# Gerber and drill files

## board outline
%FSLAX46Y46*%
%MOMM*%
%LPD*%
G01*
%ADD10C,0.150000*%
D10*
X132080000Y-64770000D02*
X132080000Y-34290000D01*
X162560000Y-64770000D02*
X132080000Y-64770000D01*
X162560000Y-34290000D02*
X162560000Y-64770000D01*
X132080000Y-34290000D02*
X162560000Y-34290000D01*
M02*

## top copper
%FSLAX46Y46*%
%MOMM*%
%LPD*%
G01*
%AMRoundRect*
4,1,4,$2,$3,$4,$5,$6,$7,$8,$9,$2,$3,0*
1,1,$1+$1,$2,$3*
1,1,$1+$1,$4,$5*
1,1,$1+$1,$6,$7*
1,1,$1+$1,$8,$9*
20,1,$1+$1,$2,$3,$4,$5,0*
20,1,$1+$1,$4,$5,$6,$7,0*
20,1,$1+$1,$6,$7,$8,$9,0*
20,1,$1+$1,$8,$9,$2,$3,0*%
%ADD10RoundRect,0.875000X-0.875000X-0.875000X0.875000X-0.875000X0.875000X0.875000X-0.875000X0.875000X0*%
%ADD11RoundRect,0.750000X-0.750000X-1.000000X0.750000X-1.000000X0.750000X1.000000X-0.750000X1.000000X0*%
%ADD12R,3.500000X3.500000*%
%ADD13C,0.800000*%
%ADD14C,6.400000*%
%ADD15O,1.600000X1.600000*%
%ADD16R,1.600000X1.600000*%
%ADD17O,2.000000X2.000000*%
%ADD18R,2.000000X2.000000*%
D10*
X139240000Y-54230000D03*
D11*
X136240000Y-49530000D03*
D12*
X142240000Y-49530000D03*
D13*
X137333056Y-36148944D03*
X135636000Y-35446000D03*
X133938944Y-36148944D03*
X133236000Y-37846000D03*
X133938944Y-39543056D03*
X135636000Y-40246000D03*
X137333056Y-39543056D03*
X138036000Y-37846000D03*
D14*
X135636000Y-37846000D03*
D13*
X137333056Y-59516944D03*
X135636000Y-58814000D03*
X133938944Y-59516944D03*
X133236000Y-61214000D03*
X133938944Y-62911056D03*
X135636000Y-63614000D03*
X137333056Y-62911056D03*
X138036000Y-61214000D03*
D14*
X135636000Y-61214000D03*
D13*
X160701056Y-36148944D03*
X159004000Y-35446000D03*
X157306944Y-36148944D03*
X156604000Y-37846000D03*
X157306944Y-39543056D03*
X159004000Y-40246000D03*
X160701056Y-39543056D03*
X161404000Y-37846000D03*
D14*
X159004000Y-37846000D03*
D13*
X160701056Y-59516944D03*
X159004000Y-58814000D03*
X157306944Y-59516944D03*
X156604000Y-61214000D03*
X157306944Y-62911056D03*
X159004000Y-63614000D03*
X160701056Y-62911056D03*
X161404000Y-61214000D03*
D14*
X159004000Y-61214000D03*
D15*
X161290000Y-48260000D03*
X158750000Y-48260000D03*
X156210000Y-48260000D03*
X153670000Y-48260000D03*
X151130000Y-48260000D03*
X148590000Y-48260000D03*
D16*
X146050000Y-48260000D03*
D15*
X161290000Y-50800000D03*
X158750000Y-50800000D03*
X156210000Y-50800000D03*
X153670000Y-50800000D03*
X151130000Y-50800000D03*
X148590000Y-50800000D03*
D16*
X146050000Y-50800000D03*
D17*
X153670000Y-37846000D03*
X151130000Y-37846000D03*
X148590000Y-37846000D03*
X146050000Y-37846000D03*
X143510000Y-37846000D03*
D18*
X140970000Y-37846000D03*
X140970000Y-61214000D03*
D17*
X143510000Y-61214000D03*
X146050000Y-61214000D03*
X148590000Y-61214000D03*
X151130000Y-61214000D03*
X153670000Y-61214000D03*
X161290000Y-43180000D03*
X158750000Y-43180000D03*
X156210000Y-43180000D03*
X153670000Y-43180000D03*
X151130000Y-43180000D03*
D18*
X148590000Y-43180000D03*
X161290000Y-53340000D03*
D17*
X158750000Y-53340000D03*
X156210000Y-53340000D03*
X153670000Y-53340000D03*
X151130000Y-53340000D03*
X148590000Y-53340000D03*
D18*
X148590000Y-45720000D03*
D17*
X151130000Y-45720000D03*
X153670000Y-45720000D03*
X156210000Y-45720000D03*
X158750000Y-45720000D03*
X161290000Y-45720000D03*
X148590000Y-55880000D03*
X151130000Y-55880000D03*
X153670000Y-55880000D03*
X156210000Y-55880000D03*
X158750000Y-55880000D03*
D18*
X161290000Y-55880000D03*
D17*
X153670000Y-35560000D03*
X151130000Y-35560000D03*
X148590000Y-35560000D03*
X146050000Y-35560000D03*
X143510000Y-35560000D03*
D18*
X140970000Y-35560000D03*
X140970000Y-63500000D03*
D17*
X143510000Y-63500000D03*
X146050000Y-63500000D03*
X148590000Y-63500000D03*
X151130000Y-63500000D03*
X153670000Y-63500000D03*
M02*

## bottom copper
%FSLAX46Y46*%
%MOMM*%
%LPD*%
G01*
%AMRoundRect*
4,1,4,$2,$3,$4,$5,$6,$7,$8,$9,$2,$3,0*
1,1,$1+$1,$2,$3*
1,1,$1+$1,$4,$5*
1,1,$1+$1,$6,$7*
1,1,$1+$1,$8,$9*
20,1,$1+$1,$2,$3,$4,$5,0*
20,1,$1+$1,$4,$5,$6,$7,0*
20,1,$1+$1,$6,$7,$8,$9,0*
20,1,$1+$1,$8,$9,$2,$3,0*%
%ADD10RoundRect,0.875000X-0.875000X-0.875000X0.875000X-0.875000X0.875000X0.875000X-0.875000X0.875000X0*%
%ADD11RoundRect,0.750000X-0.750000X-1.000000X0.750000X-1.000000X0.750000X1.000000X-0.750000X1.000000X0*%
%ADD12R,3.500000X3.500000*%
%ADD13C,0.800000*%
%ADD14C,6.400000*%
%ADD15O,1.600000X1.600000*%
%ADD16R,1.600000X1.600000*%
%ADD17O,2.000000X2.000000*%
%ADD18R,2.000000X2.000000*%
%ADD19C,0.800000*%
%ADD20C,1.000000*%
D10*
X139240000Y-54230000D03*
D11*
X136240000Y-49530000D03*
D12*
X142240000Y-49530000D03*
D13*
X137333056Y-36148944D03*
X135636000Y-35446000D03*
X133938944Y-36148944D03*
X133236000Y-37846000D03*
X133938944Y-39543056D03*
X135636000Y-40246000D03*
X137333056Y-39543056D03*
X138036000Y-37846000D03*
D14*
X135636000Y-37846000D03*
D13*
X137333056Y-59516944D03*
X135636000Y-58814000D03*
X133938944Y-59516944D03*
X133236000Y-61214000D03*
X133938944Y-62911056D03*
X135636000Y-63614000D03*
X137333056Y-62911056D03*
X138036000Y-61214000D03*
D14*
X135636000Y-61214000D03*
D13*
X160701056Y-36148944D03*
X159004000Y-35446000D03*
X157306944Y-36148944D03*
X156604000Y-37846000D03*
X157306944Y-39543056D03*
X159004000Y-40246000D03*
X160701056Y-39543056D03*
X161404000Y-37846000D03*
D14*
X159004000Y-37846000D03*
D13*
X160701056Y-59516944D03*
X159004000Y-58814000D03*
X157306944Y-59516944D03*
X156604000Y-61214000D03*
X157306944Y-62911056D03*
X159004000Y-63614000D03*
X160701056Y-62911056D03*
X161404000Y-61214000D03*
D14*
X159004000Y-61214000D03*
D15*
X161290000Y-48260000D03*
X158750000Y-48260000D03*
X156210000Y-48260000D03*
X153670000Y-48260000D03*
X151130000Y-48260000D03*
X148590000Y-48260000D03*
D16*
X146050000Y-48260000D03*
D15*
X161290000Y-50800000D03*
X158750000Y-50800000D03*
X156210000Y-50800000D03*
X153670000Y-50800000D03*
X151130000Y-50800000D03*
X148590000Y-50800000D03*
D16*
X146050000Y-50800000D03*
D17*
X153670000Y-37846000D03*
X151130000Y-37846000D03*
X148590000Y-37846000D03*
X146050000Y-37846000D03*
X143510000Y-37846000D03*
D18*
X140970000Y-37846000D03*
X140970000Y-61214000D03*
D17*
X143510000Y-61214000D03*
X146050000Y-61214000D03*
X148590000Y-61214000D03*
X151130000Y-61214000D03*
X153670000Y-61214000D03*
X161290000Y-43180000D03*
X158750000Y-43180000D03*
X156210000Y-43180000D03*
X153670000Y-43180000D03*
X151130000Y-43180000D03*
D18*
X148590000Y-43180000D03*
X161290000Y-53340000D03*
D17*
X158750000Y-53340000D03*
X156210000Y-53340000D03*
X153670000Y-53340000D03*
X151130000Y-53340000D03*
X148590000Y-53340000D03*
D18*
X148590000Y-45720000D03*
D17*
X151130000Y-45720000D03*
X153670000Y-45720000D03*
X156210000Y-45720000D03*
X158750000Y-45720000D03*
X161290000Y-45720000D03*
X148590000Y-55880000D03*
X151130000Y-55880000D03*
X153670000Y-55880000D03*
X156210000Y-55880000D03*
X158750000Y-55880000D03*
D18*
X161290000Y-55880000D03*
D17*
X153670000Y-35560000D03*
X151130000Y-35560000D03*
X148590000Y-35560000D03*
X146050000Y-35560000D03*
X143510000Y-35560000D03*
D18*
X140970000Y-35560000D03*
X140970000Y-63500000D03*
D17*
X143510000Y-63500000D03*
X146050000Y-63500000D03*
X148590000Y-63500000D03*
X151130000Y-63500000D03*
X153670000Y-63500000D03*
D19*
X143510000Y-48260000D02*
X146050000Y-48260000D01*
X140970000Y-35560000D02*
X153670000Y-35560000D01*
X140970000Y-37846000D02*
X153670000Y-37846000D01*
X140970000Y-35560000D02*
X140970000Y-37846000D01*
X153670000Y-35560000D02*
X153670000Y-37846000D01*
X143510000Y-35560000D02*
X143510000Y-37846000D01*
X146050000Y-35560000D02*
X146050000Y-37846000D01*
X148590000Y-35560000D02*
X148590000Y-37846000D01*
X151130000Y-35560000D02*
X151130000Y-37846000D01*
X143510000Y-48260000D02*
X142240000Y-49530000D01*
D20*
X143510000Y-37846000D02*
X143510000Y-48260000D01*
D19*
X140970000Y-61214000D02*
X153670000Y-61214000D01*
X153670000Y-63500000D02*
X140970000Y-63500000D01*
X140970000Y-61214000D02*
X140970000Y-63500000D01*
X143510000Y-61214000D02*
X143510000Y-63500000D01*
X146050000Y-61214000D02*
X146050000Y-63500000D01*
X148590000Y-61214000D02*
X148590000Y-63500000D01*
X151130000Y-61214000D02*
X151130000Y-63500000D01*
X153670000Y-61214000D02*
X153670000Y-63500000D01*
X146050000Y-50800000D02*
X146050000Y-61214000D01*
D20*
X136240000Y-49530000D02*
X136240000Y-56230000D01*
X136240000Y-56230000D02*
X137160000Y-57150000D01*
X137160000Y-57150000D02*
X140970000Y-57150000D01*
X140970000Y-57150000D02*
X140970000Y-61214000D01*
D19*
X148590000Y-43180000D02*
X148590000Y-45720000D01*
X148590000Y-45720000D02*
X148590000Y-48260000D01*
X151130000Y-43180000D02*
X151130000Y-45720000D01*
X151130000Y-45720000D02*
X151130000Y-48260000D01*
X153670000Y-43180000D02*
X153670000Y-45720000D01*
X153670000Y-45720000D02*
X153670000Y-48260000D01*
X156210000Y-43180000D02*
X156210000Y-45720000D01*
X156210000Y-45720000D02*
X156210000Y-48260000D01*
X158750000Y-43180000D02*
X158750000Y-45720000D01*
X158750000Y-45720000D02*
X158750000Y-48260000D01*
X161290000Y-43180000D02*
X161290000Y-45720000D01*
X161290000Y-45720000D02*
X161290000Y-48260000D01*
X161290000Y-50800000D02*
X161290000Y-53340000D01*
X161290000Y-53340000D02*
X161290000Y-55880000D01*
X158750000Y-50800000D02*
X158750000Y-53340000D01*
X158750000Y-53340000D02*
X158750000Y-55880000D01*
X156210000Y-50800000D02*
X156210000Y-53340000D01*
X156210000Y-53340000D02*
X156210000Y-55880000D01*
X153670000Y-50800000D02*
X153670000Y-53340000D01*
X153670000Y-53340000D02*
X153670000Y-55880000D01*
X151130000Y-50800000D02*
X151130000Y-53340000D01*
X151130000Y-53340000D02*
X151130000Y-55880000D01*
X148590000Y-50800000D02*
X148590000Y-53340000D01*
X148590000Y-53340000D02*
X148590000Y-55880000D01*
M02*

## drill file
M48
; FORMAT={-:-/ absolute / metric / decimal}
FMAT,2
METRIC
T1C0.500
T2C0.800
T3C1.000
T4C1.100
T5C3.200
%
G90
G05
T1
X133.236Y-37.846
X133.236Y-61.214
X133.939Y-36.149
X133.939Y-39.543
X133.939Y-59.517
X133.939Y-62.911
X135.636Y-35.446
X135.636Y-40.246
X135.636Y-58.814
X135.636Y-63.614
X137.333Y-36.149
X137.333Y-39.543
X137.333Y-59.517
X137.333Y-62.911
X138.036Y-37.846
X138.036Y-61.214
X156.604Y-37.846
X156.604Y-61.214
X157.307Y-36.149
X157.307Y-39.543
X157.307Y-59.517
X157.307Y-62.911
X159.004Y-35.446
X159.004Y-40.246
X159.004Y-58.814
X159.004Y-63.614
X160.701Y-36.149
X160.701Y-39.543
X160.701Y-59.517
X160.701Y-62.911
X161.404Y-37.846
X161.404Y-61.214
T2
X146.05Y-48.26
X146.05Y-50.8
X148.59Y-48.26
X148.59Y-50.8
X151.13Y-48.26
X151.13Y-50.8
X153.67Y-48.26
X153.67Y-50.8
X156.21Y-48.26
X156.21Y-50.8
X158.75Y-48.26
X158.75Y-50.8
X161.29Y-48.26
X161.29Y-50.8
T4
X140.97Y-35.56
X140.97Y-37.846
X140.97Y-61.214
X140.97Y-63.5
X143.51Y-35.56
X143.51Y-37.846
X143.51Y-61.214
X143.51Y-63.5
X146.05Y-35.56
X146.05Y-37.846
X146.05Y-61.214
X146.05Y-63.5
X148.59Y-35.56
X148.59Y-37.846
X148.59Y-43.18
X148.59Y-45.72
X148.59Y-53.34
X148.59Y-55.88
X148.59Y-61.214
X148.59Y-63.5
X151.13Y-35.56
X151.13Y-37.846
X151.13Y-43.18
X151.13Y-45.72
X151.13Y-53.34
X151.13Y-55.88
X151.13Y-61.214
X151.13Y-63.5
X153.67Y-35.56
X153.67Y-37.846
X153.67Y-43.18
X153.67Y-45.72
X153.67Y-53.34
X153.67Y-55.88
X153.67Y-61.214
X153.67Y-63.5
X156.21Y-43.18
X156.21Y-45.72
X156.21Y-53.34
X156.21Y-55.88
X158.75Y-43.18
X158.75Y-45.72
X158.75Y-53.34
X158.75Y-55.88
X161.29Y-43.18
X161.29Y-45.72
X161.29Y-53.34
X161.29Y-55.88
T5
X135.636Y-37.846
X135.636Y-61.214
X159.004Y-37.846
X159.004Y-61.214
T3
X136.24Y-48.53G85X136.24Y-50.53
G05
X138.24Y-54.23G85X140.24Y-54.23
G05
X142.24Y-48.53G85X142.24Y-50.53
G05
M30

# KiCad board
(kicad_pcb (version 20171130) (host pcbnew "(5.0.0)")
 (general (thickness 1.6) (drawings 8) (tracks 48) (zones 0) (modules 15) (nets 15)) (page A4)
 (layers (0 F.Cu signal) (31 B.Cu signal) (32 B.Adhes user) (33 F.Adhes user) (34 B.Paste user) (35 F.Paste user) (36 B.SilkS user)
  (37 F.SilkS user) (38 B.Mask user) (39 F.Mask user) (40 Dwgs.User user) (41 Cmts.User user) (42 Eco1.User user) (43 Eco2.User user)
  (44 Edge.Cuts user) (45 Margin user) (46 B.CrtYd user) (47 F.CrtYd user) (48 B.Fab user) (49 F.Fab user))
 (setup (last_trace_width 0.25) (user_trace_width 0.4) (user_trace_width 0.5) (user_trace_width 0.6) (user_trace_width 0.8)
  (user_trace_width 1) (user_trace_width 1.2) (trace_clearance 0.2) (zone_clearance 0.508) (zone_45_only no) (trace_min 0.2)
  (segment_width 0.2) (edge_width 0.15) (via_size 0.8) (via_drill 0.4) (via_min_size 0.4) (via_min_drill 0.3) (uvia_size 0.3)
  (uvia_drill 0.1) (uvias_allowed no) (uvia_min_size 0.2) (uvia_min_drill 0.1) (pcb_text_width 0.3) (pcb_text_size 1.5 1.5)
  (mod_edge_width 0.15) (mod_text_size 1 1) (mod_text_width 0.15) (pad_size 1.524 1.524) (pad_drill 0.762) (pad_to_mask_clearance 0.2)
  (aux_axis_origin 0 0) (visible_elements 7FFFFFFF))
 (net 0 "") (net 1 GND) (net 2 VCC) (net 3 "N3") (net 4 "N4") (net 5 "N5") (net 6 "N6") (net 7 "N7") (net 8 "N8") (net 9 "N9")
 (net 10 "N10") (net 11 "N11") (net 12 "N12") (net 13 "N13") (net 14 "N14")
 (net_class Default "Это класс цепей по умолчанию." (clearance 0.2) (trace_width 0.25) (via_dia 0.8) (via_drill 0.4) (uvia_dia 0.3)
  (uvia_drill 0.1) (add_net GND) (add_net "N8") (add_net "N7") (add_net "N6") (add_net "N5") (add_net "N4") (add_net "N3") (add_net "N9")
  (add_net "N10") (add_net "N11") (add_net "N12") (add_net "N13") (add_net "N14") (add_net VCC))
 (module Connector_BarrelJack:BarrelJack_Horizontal (layer F.Cu) (at 142.24 49.53)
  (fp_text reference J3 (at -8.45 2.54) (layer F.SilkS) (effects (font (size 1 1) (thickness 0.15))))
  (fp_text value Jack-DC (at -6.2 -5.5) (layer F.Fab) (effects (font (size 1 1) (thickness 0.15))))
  (pad 3 thru_hole roundrect (at -3 4.7) (size 3.5 3.5) (drill oval 3 1) (layers *.Cu *.Mask) (roundrect_rratio 0.25))
  (pad 2 thru_hole roundrect (at -6 0) (size 3 3.5) (drill oval 1 3) (layers *.Cu *.Mask) (roundrect_rratio 0.25) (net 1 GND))
  (pad 1 thru_hole rect (at 0 0) (size 3.5 3.5) (drill oval 1 3) (layers *.Cu *.Mask) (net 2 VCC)))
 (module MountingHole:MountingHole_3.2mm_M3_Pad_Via (layer F.Cu) (at 135.636 37.846)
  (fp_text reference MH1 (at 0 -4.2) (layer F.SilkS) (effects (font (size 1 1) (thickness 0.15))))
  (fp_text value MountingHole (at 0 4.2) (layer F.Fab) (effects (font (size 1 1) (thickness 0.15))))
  (pad 1 thru_hole circle (at 1.697056 -1.697056) (size 0.8 0.8) (drill 0.5) (layers *.Cu *.Mask))
  (pad 1 thru_hole circle (at 0 -2.4) (size 0.8 0.8) (drill 0.5) (layers *.Cu *.Mask))
  (pad 1 thru_hole circle (at -1.697056 -1.697056) (size 0.8 0.8) (drill 0.5) (layers *.Cu *.Mask))
  (pad 1 thru_hole circle (at -2.4 0) (size 0.8 0.8) (drill 0.5) (layers *.Cu *.Mask))
  (pad 1 thru_hole circle (at -1.697056 1.697056) (size 0.8 0.8) (drill 0.5) (layers *.Cu *.Mask))
  (pad 1 thru_hole circle (at 0 2.4) (size 0.8 0.8) (drill 0.5) (layers *.Cu *.Mask))
  (pad 1 thru_hole circle (at 1.697056 1.697056) (size 0.8 0.8) (drill 0.5) (layers *.Cu *.Mask))
  (pad 1 thru_hole circle (at 2.4 0) (size 0.8 0.8) (drill 0.5) (layers *.Cu *.Mask))
  (pad 1 thru_hole circle (at 0 0) (size 6.4 6.4) (drill 3.2) (layers *.Cu *.Mask)))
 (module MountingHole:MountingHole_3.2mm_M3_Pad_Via (layer F.Cu) (at 135.636 61.214)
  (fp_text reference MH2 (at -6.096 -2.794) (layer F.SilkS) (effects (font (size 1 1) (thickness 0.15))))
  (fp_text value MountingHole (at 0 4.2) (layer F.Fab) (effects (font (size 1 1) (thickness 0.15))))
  (pad 1 thru_hole circle (at 1.697056 -1.697056) (size 0.8 0.8) (drill 0.5) (layers *.Cu *.Mask))
  (pad 1 thru_hole circle (at 0 -2.4) (size 0.8 0.8) (drill 0.5) (layers *.Cu *.Mask))
  (pad 1 thru_hole circle (at -1.697056 -1.697056) (size 0.8 0.8) (drill 0.5) (layers *.Cu *.Mask))
  (pad 1 thru_hole circle (at -2.4 0) (size 0.8 0.8) (drill 0.5) (layers *.Cu *.Mask))
  (pad 1 thru_hole circle (at -1.697056 1.697056) (size 0.8 0.8) (drill 0.5) (layers *.Cu *.Mask))
  (pad 1 thru_hole circle (at 0 2.4) (size 0.8 0.8) (drill 0.5) (layers *.Cu *.Mask))
  (pad 1 thru_hole circle (at 1.697056 1.697056) (size 0.8 0.8) (drill 0.5) (layers *.Cu *.Mask))
  (pad 1 thru_hole circle (at 2.4 0) (size 0.8 0.8) (drill 0.5) (layers *.Cu *.Mask))
  (pad 1 thru_hole circle (at 0 0) (size 6.4 6.4) (drill 3.2) (layers *.Cu *.Mask)))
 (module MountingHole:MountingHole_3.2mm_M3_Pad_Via (layer F.Cu) (at 159.004 37.846)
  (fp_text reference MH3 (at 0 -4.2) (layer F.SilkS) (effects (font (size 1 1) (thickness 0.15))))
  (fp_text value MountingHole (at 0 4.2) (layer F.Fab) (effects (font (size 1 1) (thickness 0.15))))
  (pad 1 thru_hole circle (at 1.697056 -1.697056) (size 0.8 0.8) (drill 0.5) (layers *.Cu *.Mask))
  (pad 1 thru_hole circle (at 0 -2.4) (size 0.8 0.8) (drill 0.5) (layers *.Cu *.Mask))
  (pad 1 thru_hole circle (at -1.697056 -1.697056) (size 0.8 0.8) (drill 0.5) (layers *.Cu *.Mask))
  (pad 1 thru_hole circle (at -2.4 0) (size 0.8 0.8) (drill 0.5) (layers *.Cu *.Mask))
  (pad 1 thru_hole circle (at -1.697056 1.697056) (size 0.8 0.8) (drill 0.5) (layers *.Cu *.Mask))
  (pad 1 thru_hole circle (at 0 2.4) (size 0.8 0.8) (drill 0.5) (layers *.Cu *.Mask))
  (pad 1 thru_hole circle (at 1.697056 1.697056) (size 0.8 0.8) (drill 0.5) (layers *.Cu *.Mask))
  (pad 1 thru_hole circle (at 2.4 0) (size 0.8 0.8) (drill 0.5) (layers *.Cu *.Mask))
  (pad 1 thru_hole circle (at 0 0) (size 6.4 6.4) (drill 3.2) (layers *.Cu *.Mask)))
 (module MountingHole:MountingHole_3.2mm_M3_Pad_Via (layer F.Cu) (at 159.004 61.214)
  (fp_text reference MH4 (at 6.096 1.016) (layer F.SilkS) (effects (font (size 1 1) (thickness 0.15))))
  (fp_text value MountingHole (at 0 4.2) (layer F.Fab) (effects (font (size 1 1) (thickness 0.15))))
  (pad 1 thru_hole circle (at 1.697056 -1.697056) (size 0.8 0.8) (drill 0.5) (layers *.Cu *.Mask))
  (pad 1 thru_hole circle (at 0 -2.4) (size 0.8 0.8) (drill 0.5) (layers *.Cu *.Mask))
  (pad 1 thru_hole circle (at -1.697056 -1.697056) (size 0.8 0.8) (drill 0.5) (layers *.Cu *.Mask))
  (pad 1 thru_hole circle (at -2.4 0) (size 0.8 0.8) (drill 0.5) (layers *.Cu *.Mask))
  (pad 1 thru_hole circle (at -1.697056 1.697056) (size 0.8 0.8) (drill 0.5) (layers *.Cu *.Mask))
  (pad 1 thru_hole circle (at 0 2.4) (size 0.8 0.8) (drill 0.5) (layers *.Cu *.Mask))
  (pad 1 thru_hole circle (at 1.697056 1.697056) (size 0.8 0.8) (drill 0.5) (layers *.Cu *.Mask))
  (pad 1 thru_hole circle (at 2.4 0) (size 0.8 0.8) (drill 0.5) (layers *.Cu *.Mask))
  (pad 1 thru_hole circle (at 0 0) (size 6.4 6.4) (drill 3.2) (layers *.Cu *.Mask)))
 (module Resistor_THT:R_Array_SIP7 (layer F.Cu) (at 146.05 48.26)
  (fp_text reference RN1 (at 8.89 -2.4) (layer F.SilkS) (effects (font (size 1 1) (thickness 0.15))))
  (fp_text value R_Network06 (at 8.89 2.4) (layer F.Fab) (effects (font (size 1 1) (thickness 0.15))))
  (pad 7 thru_hole oval (at 15.24 0) (size 1.6 1.6) (drill 0.8) (layers *.Cu *.Mask) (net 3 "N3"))
  (pad 6 thru_hole oval (at 12.7 0) (size 1.6 1.6) (drill 0.8) (layers *.Cu *.Mask) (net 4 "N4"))
  (pad 5 thru_hole oval (at 10.16 0) (size 1.6 1.6) (drill 0.8) (layers *.Cu *.Mask) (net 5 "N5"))
  (pad 4 thru_hole oval (at 7.62 0) (size 1.6 1.6) (drill 0.8) (layers *.Cu *.Mask) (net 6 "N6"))
  (pad 3 thru_hole oval (at 5.08 0) (size 1.6 1.6) (drill 0.8) (layers *.Cu *.Mask) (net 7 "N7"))
  (pad 2 thru_hole oval (at 2.54 0) (size 1.6 1.6) (drill 0.8) (layers *.Cu *.Mask) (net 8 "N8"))
  (pad 1 thru_hole rect (at 0 0) (size 1.6 1.6) (drill 0.8) (layers *.Cu *.Mask) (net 2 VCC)))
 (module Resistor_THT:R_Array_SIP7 (layer F.Cu) (at 146.05 50.8)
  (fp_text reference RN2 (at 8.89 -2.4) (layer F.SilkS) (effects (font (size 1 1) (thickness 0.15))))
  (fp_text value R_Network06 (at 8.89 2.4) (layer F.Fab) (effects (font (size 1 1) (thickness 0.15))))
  (pad 7 thru_hole oval (at 15.24 0) (size 1.6 1.6) (drill 0.8) (layers *.Cu *.Mask) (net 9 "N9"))
  (pad 6 thru_hole oval (at 12.7 0) (size 1.6 1.6) (drill 0.8) (layers *.Cu *.Mask) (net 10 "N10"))
  (pad 5 thru_hole oval (at 10.16 0) (size 1.6 1.6) (drill 0.8) (layers *.Cu *.Mask) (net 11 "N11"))
  (pad 4 thru_hole oval (at 7.62 0) (size 1.6 1.6) (drill 0.8) (layers *.Cu *.Mask) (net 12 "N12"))
  (pad 3 thru_hole oval (at 5.08 0) (size 1.6 1.6) (drill 0.8) (layers *.Cu *.Mask) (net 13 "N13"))
  (pad 2 thru_hole oval (at 2.54 0) (size 1.6 1.6) (drill 0.8) (layers *.Cu *.Mask) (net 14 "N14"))
  (pad 1 thru_hole rect (at 0 0) (size 1.6 1.6) (drill 0.8) (layers *.Cu *.Mask) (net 1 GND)))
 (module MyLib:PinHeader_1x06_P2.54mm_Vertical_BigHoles (layer F.Cu) (at 140.97 37.846 90)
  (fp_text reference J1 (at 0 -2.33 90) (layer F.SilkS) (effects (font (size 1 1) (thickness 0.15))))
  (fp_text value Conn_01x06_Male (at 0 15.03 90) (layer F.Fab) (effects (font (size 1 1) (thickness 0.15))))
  (pad 6 thru_hole oval (at 0 12.7 90) (size 2 2) (drill 1.1) (layers *.Cu *.Mask) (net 2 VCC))
  (pad 5 thru_hole oval (at 0 10.16 90) (size 2 2) (drill 1.1) (layers *.Cu *.Mask) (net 2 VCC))
  (pad 4 thru_hole oval (at 0 7.62 90) (size 2 2) (drill 1.1) (layers *.Cu *.Mask) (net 2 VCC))
  (pad 3 thru_hole oval (at 0 5.08 90) (size 2 2) (drill 1.1) (layers *.Cu *.Mask) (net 2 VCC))
  (pad 2 thru_hole oval (at 0 2.54 90) (size 2 2) (drill 1.1) (layers *.Cu *.Mask) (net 2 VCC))
  (pad 1 thru_hole rect (at 0 0 90) (size 2 2) (drill 1.1) (layers *.Cu *.Mask) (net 2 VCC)))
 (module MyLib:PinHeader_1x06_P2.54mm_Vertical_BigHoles (layer F.Cu) (at 140.97 61.214 90)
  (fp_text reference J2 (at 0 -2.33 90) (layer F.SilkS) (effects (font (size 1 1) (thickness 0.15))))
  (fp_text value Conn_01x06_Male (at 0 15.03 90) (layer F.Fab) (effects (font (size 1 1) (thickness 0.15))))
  (pad 1 thru_hole rect (at 0 0 90) (size 2 2) (drill 1.1) (layers *.Cu *.Mask) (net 1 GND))
  (pad 2 thru_hole oval (at 0 2.54 90) (size 2 2) (drill 1.1) (layers *.Cu *.Mask) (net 1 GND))
  (pad 3 thru_hole oval (at 0 5.08 90) (size 2 2) (drill 1.1) (layers *.Cu *.Mask) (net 1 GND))
  (pad 4 thru_hole oval (at 0 7.62 90) (size 2 2) (drill 1.1) (layers *.Cu *.Mask) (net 1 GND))
  (pad 5 thru_hole oval (at 0 10.16 90) (size 2 2) (drill 1.1) (layers *.Cu *.Mask) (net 1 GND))
  (pad 6 thru_hole oval (at 0 12.7 90) (size 2 2) (drill 1.1) (layers *.Cu *.Mask) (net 1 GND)))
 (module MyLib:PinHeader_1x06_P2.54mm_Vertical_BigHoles (layer F.Cu) (at 148.59 43.18 90)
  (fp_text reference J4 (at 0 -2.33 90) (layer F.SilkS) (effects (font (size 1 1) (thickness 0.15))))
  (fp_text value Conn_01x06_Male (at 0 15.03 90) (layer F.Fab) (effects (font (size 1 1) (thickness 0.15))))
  (pad 6 thru_hole oval (at 0 12.7 90) (size 2 2) (drill 1.1) (layers *.Cu *.Mask) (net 3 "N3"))
  (pad 5 thru_hole oval (at 0 10.16 90) (size 2 2) (drill 1.1) (layers *.Cu *.Mask) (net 4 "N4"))
  (pad 4 thru_hole oval (at 0 7.62 90) (size 2 2) (drill 1.1) (layers *.Cu *.Mask) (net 5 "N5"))
  (pad 3 thru_hole oval (at 0 5.08 90) (size 2 2) (drill 1.1) (layers *.Cu *.Mask) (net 6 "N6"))
  (pad 2 thru_hole oval (at 0 2.54 90) (size 2 2) (drill 1.1) (layers *.Cu *.Mask) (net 7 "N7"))
  (pad 1 thru_hole rect (at 0 0 90) (size 2 2) (drill 1.1) (layers *.Cu *.Mask) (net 8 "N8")))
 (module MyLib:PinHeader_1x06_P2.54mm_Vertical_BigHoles (layer F.Cu) (at 161.29 53.34 270)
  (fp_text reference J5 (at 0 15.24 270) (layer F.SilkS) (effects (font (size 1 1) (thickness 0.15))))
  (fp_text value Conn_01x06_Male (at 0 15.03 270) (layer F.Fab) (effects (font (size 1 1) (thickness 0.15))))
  (pad 1 thru_hole rect (at 0 0 270) (size 2 2) (drill 1.1) (layers *.Cu *.Mask) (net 9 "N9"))
  (pad 2 thru_hole oval (at 0 2.54 270) (size 2 2) (drill 1.1) (layers *.Cu *.Mask) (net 10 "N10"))
  (pad 3 thru_hole oval (at 0 5.08 270) (size 2 2) (drill 1.1) (layers *.Cu *.Mask) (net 11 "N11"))
  (pad 4 thru_hole oval (at 0 7.62 270) (size 2 2) (drill 1.1) (layers *.Cu *.Mask) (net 12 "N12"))
  (pad 5 thru_hole oval (at 0 10.16 270) (size 2 2) (drill 1.1) (layers *.Cu *.Mask) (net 13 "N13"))
  (pad 6 thru_hole oval (at 0 12.7 270) (size 2 2) (drill 1.1) (layers *.Cu *.Mask) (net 14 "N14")))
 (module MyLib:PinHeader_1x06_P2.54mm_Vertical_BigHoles (layer F.Cu) (at 148.59 45.72 90)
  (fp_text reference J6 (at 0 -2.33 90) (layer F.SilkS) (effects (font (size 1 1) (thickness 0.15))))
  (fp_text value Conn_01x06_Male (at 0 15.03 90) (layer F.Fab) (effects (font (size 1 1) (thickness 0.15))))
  (pad 1 thru_hole rect (at 0 0 90) (size 2 2) (drill 1.1) (layers *.Cu *.Mask) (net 8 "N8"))
  (pad 2 thru_hole oval (at 0 2.54 90) (size 2 2) (drill 1.1) (layers *.Cu *.Mask) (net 7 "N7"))
  (pad 3 thru_hole oval (at 0 5.08 90) (size 2 2) (drill 1.1) (layers *.Cu *.Mask) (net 6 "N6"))
  (pad 4 thru_hole oval (at 0 7.62 90) (size 2 2) (drill 1.1) (layers *.Cu *.Mask) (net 5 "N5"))
  (pad 5 thru_hole oval (at 0 10.16 90) (size 2 2) (drill 1.1) (layers *.Cu *.Mask) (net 4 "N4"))
  (pad 6 thru_hole oval (at 0 12.7 90) (size 2 2) (drill 1.1) (layers *.Cu *.Mask) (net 3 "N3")))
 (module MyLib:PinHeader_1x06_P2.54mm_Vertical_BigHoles (layer F.Cu) (at 161.29 55.88 270)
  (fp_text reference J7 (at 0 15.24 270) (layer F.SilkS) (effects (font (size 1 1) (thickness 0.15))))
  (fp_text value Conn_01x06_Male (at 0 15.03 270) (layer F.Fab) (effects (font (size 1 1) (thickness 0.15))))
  (pad 6 thru_hole oval (at 0 12.7 270) (size 2 2) (drill 1.1) (layers *.Cu *.Mask) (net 14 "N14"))
  (pad 5 thru_hole oval (at 0 10.16 270) (size 2 2) (drill 1.1) (layers *.Cu *.Mask) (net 13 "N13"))
  (pad 4 thru_hole oval (at 0 7.62 270) (size 2 2) (drill 1.1) (layers *.Cu *.Mask) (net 12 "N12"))
  (pad 3 thru_hole oval (at 0 5.08 270) (size 2 2) (drill 1.1) (layers *.Cu *.Mask) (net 11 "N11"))
  (pad 2 thru_hole oval (at 0 2.54 270) (size 2 2) (drill 1.1) (layers *.Cu *.Mask) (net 10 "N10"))
  (pad 1 thru_hole rect (at 0 0 270) (size 2 2) (drill 1.1) (layers *.Cu *.Mask) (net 9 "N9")))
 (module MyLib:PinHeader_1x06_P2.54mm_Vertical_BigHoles (layer F.Cu) (at 140.97 35.56 90)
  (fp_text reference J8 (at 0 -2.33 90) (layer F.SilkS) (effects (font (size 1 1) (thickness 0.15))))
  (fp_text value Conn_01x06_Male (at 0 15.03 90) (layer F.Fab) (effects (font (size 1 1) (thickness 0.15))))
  (pad 6 thru_hole oval (at 0 12.7 90) (size 2 2) (drill 1.1) (layers *.Cu *.Mask) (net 2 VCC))
  (pad 5 thru_hole oval (at 0 10.16 90) (size 2 2) (drill 1.1) (layers *.Cu *.Mask) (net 2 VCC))
  (pad 4 thru_hole oval (at 0 7.62 90) (size 2 2) (drill 1.1) (layers *.Cu *.Mask) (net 2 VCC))
  (pad 3 thru_hole oval (at 0 5.08 90) (size 2 2) (drill 1.1) (layers *.Cu *.Mask) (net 2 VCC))
  (pad 2 thru_hole oval (at 0 2.54 90) (size 2 2) (drill 1.1) (layers *.Cu *.Mask) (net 2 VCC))
  (pad 1 thru_hole rect (at 0 0 90) (size 2 2) (drill 1.1) (layers *.Cu *.Mask) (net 2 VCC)))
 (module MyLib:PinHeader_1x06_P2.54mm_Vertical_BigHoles (layer F.Cu) (at 140.97 63.5 90)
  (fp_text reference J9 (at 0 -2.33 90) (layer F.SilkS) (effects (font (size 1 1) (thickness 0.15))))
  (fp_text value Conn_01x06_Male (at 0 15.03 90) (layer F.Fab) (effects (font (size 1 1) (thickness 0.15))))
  (pad 1 thru_hole rect (at 0 0 90) (size 2 2) (drill 1.1) (layers *.Cu *.Mask) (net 1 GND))
  (pad 2 thru_hole oval (at 0 2.54 90) (size 2 2) (drill 1.1) (layers *.Cu *.Mask) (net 1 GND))
  (pad 3 thru_hole oval (at 0 5.08 90) (size 2 2) (drill 1.1) (layers *.Cu *.Mask) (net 1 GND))
  (pad 4 thru_hole oval (at 0 7.62 90) (size 2 2) (drill 1.1) (layers *.Cu *.Mask) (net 1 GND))
  (pad 5 thru_hole oval (at 0 10.16 90) (size 2 2) (drill 1.1) (layers *.Cu *.Mask) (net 1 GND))
  (pad 6 thru_hole oval (at 0 12.7 90) (size 2 2) (drill 1.1) (layers *.Cu *.Mask) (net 1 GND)))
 (gr_line (start 132.08 64.77) (end 132.08 34.29) (layer Edge.Cuts) (width 0.15))
 (gr_line (start 162.56 64.77) (end 132.08 64.77) (layer Edge.Cuts) (width 0.15))
 (gr_line (start 162.56 34.29) (end 162.56 64.77) (layer Edge.Cuts) (width 0.15))
 (gr_line (start 132.08 34.29) (end 162.56 34.29) (layer Edge.Cuts) (width 0.15))
 (segment (start 143.51 48.26) (end 146.05 48.26) (width 0.8) (layer B.Cu) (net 2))
 (segment (start 140.97 35.56) (end 153.67 35.56) (width 0.8) (layer B.Cu) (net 2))
 (segment (start 140.97 37.846) (end 153.67 37.846) (width 0.8) (layer B.Cu) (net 2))
 (segment (start 140.97 35.56) (end 140.97 37.846) (width 0.8) (layer B.Cu) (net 2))
 (segment (start 153.67 35.56) (end 153.67 37.846) (width 0.8) (layer B.Cu) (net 2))
 (segment (start 143.51 35.56) (end 143.51 37.846) (width 0.8) (layer B.Cu) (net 2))
 (segment (start 146.05 35.56) (end 146.05 37.846) (width 0.8) (layer B.Cu) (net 2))
 (segment (start 148.59 35.56) (end 148.59 37.846) (width 0.8) (layer B.Cu) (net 2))
 (segment (start 151.13 35.56) (end 151.13 37.846) (width 0.8) (layer B.Cu) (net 2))
 (segment (start 143.51 48.26) (end 142.24 49.53) (width 0.8) (layer B.Cu) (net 2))
 (segment (start 143.51 37.846) (end 143.51 48.26) (width 1) (layer B.Cu) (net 2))
 (segment (start 140.97 61.214) (end 153.67 61.214) (width 0.8) (layer B.Cu) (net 1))
 (segment (start 153.67 63.5) (end 140.97 63.5) (width 0.8) (layer B.Cu) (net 1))
 (segment (start 140.97 61.214) (end 140.97 63.5) (width 0.8) (layer B.Cu) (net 1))
 (segment (start 143.51 61.214) (end 143.51 63.5) (width 0.8) (layer B.Cu) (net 1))
 (segment (start 146.05 61.214) (end 146.05 63.5) (width 0.8) (layer B.Cu) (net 1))
 (segment (start 148.59 61.214) (end 148.59 63.5) (width 0.8) (layer B.Cu) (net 1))
 (segment (start 151.13 61.214) (end 151.13 63.5) (width 0.8) (layer B.Cu) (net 1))
 (segment (start 153.67 61.214) (end 153.67 63.5) (width 0.8) (layer B.Cu) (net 1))
 (segment (start 146.05 50.8) (end 146.05 61.214) (width 0.8) (layer B.Cu) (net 1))
 (segment (start 136.24 49.53) (end 136.24 56.23) (width 1) (layer B.Cu) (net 1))
 (segment (start 136.24 56.23) (end 137.16 57.15) (width 1) (layer B.Cu) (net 1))
 (segment (start 137.16 57.15) (end 140.97 57.15) (width 1) (layer B.Cu) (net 1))
 (segment (start 140.97 57.15) (end 140.97 61.214) (width 1) (layer B.Cu) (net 1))
 (segment (start 148.59 43.18) (end 148.59 45.72) (width 0.8) (layer B.Cu) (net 8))
 (segment (start 148.59 45.72) (end 148.59 48.26) (width 0.8) (layer B.Cu) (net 8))
 (segment (start 151.13 43.18) (end 151.13 45.72) (width 0.8) (layer B.Cu) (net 7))
 (segment (start 151.13 45.72) (end 151.13 48.26) (width 0.8) (layer B.Cu) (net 7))
 (segment (start 153.67 43.18) (end 153.67 45.72) (width 0.8) (layer B.Cu) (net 6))
 (segment (start 153.67 45.72) (end 153.67 48.26) (width 0.8) (layer B.Cu) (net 6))
 (segment (start 156.21 43.18) (end 156.21 45.72) (width 0.8) (layer B.Cu) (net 5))
 (segment (start 156.21 45.72) (end 156.21 48.26) (width 0.8) (layer B.Cu) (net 5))
 (segment (start 158.75 43.18) (end 158.75 45.72) (width 0.8) (layer B.Cu) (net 4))
 (segment (start 158.75 45.72) (end 158.75 48.26) (width 0.8) (layer B.Cu) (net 4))
 (segment (start 161.29 43.18) (end 161.29 45.72) (width 0.8) (layer B.Cu) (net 3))
 (segment (start 161.29 45.72) (end 161.29 48.26) (width 0.8) (layer B.Cu) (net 3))
 (segment (start 161.29 50.8) (end 161.29 53.34) (width 0.8) (layer B.Cu) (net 9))
 (segment (start 161.29 53.34) (end 161.29 55.88) (width 0.8) (layer B.Cu) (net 9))
 (segment (start 158.75 50.8) (end 158.75 53.34) (width 0.8) (layer B.Cu) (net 10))
 (segment (start 158.75 53.34) (end 158.75 55.88) (width 0.8) (layer B.Cu) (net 10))
 (segment (start 156.21 50.8) (end 156.21 53.34) (width 0.8) (layer B.Cu) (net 11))
 (segment (start 156.21 53.34) (end 156.21 55.88) (width 0.8) (layer B.Cu) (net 11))
 (segment (start 153.67 50.8) (end 153.67 53.34) (width 0.8) (layer B.Cu) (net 12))
 (segment (start 153.67 53.34) (end 153.67 55.88) (width 0.8) (layer B.Cu) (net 12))
 (segment (start 151.13 50.8) (end 151.13 53.34) (width 0.8) (layer B.Cu) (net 13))
 (segment (start 151.13 53.34) (end 151.13 55.88) (width 0.8) (layer B.Cu) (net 13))
 (segment (start 148.59 50.8) (end 148.59 53.34) (width 0.8) (layer B.Cu) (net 14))
 (segment (start 148.59 53.34) (end 148.59 55.88) (width 0.8) (layer B.Cu) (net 14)))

